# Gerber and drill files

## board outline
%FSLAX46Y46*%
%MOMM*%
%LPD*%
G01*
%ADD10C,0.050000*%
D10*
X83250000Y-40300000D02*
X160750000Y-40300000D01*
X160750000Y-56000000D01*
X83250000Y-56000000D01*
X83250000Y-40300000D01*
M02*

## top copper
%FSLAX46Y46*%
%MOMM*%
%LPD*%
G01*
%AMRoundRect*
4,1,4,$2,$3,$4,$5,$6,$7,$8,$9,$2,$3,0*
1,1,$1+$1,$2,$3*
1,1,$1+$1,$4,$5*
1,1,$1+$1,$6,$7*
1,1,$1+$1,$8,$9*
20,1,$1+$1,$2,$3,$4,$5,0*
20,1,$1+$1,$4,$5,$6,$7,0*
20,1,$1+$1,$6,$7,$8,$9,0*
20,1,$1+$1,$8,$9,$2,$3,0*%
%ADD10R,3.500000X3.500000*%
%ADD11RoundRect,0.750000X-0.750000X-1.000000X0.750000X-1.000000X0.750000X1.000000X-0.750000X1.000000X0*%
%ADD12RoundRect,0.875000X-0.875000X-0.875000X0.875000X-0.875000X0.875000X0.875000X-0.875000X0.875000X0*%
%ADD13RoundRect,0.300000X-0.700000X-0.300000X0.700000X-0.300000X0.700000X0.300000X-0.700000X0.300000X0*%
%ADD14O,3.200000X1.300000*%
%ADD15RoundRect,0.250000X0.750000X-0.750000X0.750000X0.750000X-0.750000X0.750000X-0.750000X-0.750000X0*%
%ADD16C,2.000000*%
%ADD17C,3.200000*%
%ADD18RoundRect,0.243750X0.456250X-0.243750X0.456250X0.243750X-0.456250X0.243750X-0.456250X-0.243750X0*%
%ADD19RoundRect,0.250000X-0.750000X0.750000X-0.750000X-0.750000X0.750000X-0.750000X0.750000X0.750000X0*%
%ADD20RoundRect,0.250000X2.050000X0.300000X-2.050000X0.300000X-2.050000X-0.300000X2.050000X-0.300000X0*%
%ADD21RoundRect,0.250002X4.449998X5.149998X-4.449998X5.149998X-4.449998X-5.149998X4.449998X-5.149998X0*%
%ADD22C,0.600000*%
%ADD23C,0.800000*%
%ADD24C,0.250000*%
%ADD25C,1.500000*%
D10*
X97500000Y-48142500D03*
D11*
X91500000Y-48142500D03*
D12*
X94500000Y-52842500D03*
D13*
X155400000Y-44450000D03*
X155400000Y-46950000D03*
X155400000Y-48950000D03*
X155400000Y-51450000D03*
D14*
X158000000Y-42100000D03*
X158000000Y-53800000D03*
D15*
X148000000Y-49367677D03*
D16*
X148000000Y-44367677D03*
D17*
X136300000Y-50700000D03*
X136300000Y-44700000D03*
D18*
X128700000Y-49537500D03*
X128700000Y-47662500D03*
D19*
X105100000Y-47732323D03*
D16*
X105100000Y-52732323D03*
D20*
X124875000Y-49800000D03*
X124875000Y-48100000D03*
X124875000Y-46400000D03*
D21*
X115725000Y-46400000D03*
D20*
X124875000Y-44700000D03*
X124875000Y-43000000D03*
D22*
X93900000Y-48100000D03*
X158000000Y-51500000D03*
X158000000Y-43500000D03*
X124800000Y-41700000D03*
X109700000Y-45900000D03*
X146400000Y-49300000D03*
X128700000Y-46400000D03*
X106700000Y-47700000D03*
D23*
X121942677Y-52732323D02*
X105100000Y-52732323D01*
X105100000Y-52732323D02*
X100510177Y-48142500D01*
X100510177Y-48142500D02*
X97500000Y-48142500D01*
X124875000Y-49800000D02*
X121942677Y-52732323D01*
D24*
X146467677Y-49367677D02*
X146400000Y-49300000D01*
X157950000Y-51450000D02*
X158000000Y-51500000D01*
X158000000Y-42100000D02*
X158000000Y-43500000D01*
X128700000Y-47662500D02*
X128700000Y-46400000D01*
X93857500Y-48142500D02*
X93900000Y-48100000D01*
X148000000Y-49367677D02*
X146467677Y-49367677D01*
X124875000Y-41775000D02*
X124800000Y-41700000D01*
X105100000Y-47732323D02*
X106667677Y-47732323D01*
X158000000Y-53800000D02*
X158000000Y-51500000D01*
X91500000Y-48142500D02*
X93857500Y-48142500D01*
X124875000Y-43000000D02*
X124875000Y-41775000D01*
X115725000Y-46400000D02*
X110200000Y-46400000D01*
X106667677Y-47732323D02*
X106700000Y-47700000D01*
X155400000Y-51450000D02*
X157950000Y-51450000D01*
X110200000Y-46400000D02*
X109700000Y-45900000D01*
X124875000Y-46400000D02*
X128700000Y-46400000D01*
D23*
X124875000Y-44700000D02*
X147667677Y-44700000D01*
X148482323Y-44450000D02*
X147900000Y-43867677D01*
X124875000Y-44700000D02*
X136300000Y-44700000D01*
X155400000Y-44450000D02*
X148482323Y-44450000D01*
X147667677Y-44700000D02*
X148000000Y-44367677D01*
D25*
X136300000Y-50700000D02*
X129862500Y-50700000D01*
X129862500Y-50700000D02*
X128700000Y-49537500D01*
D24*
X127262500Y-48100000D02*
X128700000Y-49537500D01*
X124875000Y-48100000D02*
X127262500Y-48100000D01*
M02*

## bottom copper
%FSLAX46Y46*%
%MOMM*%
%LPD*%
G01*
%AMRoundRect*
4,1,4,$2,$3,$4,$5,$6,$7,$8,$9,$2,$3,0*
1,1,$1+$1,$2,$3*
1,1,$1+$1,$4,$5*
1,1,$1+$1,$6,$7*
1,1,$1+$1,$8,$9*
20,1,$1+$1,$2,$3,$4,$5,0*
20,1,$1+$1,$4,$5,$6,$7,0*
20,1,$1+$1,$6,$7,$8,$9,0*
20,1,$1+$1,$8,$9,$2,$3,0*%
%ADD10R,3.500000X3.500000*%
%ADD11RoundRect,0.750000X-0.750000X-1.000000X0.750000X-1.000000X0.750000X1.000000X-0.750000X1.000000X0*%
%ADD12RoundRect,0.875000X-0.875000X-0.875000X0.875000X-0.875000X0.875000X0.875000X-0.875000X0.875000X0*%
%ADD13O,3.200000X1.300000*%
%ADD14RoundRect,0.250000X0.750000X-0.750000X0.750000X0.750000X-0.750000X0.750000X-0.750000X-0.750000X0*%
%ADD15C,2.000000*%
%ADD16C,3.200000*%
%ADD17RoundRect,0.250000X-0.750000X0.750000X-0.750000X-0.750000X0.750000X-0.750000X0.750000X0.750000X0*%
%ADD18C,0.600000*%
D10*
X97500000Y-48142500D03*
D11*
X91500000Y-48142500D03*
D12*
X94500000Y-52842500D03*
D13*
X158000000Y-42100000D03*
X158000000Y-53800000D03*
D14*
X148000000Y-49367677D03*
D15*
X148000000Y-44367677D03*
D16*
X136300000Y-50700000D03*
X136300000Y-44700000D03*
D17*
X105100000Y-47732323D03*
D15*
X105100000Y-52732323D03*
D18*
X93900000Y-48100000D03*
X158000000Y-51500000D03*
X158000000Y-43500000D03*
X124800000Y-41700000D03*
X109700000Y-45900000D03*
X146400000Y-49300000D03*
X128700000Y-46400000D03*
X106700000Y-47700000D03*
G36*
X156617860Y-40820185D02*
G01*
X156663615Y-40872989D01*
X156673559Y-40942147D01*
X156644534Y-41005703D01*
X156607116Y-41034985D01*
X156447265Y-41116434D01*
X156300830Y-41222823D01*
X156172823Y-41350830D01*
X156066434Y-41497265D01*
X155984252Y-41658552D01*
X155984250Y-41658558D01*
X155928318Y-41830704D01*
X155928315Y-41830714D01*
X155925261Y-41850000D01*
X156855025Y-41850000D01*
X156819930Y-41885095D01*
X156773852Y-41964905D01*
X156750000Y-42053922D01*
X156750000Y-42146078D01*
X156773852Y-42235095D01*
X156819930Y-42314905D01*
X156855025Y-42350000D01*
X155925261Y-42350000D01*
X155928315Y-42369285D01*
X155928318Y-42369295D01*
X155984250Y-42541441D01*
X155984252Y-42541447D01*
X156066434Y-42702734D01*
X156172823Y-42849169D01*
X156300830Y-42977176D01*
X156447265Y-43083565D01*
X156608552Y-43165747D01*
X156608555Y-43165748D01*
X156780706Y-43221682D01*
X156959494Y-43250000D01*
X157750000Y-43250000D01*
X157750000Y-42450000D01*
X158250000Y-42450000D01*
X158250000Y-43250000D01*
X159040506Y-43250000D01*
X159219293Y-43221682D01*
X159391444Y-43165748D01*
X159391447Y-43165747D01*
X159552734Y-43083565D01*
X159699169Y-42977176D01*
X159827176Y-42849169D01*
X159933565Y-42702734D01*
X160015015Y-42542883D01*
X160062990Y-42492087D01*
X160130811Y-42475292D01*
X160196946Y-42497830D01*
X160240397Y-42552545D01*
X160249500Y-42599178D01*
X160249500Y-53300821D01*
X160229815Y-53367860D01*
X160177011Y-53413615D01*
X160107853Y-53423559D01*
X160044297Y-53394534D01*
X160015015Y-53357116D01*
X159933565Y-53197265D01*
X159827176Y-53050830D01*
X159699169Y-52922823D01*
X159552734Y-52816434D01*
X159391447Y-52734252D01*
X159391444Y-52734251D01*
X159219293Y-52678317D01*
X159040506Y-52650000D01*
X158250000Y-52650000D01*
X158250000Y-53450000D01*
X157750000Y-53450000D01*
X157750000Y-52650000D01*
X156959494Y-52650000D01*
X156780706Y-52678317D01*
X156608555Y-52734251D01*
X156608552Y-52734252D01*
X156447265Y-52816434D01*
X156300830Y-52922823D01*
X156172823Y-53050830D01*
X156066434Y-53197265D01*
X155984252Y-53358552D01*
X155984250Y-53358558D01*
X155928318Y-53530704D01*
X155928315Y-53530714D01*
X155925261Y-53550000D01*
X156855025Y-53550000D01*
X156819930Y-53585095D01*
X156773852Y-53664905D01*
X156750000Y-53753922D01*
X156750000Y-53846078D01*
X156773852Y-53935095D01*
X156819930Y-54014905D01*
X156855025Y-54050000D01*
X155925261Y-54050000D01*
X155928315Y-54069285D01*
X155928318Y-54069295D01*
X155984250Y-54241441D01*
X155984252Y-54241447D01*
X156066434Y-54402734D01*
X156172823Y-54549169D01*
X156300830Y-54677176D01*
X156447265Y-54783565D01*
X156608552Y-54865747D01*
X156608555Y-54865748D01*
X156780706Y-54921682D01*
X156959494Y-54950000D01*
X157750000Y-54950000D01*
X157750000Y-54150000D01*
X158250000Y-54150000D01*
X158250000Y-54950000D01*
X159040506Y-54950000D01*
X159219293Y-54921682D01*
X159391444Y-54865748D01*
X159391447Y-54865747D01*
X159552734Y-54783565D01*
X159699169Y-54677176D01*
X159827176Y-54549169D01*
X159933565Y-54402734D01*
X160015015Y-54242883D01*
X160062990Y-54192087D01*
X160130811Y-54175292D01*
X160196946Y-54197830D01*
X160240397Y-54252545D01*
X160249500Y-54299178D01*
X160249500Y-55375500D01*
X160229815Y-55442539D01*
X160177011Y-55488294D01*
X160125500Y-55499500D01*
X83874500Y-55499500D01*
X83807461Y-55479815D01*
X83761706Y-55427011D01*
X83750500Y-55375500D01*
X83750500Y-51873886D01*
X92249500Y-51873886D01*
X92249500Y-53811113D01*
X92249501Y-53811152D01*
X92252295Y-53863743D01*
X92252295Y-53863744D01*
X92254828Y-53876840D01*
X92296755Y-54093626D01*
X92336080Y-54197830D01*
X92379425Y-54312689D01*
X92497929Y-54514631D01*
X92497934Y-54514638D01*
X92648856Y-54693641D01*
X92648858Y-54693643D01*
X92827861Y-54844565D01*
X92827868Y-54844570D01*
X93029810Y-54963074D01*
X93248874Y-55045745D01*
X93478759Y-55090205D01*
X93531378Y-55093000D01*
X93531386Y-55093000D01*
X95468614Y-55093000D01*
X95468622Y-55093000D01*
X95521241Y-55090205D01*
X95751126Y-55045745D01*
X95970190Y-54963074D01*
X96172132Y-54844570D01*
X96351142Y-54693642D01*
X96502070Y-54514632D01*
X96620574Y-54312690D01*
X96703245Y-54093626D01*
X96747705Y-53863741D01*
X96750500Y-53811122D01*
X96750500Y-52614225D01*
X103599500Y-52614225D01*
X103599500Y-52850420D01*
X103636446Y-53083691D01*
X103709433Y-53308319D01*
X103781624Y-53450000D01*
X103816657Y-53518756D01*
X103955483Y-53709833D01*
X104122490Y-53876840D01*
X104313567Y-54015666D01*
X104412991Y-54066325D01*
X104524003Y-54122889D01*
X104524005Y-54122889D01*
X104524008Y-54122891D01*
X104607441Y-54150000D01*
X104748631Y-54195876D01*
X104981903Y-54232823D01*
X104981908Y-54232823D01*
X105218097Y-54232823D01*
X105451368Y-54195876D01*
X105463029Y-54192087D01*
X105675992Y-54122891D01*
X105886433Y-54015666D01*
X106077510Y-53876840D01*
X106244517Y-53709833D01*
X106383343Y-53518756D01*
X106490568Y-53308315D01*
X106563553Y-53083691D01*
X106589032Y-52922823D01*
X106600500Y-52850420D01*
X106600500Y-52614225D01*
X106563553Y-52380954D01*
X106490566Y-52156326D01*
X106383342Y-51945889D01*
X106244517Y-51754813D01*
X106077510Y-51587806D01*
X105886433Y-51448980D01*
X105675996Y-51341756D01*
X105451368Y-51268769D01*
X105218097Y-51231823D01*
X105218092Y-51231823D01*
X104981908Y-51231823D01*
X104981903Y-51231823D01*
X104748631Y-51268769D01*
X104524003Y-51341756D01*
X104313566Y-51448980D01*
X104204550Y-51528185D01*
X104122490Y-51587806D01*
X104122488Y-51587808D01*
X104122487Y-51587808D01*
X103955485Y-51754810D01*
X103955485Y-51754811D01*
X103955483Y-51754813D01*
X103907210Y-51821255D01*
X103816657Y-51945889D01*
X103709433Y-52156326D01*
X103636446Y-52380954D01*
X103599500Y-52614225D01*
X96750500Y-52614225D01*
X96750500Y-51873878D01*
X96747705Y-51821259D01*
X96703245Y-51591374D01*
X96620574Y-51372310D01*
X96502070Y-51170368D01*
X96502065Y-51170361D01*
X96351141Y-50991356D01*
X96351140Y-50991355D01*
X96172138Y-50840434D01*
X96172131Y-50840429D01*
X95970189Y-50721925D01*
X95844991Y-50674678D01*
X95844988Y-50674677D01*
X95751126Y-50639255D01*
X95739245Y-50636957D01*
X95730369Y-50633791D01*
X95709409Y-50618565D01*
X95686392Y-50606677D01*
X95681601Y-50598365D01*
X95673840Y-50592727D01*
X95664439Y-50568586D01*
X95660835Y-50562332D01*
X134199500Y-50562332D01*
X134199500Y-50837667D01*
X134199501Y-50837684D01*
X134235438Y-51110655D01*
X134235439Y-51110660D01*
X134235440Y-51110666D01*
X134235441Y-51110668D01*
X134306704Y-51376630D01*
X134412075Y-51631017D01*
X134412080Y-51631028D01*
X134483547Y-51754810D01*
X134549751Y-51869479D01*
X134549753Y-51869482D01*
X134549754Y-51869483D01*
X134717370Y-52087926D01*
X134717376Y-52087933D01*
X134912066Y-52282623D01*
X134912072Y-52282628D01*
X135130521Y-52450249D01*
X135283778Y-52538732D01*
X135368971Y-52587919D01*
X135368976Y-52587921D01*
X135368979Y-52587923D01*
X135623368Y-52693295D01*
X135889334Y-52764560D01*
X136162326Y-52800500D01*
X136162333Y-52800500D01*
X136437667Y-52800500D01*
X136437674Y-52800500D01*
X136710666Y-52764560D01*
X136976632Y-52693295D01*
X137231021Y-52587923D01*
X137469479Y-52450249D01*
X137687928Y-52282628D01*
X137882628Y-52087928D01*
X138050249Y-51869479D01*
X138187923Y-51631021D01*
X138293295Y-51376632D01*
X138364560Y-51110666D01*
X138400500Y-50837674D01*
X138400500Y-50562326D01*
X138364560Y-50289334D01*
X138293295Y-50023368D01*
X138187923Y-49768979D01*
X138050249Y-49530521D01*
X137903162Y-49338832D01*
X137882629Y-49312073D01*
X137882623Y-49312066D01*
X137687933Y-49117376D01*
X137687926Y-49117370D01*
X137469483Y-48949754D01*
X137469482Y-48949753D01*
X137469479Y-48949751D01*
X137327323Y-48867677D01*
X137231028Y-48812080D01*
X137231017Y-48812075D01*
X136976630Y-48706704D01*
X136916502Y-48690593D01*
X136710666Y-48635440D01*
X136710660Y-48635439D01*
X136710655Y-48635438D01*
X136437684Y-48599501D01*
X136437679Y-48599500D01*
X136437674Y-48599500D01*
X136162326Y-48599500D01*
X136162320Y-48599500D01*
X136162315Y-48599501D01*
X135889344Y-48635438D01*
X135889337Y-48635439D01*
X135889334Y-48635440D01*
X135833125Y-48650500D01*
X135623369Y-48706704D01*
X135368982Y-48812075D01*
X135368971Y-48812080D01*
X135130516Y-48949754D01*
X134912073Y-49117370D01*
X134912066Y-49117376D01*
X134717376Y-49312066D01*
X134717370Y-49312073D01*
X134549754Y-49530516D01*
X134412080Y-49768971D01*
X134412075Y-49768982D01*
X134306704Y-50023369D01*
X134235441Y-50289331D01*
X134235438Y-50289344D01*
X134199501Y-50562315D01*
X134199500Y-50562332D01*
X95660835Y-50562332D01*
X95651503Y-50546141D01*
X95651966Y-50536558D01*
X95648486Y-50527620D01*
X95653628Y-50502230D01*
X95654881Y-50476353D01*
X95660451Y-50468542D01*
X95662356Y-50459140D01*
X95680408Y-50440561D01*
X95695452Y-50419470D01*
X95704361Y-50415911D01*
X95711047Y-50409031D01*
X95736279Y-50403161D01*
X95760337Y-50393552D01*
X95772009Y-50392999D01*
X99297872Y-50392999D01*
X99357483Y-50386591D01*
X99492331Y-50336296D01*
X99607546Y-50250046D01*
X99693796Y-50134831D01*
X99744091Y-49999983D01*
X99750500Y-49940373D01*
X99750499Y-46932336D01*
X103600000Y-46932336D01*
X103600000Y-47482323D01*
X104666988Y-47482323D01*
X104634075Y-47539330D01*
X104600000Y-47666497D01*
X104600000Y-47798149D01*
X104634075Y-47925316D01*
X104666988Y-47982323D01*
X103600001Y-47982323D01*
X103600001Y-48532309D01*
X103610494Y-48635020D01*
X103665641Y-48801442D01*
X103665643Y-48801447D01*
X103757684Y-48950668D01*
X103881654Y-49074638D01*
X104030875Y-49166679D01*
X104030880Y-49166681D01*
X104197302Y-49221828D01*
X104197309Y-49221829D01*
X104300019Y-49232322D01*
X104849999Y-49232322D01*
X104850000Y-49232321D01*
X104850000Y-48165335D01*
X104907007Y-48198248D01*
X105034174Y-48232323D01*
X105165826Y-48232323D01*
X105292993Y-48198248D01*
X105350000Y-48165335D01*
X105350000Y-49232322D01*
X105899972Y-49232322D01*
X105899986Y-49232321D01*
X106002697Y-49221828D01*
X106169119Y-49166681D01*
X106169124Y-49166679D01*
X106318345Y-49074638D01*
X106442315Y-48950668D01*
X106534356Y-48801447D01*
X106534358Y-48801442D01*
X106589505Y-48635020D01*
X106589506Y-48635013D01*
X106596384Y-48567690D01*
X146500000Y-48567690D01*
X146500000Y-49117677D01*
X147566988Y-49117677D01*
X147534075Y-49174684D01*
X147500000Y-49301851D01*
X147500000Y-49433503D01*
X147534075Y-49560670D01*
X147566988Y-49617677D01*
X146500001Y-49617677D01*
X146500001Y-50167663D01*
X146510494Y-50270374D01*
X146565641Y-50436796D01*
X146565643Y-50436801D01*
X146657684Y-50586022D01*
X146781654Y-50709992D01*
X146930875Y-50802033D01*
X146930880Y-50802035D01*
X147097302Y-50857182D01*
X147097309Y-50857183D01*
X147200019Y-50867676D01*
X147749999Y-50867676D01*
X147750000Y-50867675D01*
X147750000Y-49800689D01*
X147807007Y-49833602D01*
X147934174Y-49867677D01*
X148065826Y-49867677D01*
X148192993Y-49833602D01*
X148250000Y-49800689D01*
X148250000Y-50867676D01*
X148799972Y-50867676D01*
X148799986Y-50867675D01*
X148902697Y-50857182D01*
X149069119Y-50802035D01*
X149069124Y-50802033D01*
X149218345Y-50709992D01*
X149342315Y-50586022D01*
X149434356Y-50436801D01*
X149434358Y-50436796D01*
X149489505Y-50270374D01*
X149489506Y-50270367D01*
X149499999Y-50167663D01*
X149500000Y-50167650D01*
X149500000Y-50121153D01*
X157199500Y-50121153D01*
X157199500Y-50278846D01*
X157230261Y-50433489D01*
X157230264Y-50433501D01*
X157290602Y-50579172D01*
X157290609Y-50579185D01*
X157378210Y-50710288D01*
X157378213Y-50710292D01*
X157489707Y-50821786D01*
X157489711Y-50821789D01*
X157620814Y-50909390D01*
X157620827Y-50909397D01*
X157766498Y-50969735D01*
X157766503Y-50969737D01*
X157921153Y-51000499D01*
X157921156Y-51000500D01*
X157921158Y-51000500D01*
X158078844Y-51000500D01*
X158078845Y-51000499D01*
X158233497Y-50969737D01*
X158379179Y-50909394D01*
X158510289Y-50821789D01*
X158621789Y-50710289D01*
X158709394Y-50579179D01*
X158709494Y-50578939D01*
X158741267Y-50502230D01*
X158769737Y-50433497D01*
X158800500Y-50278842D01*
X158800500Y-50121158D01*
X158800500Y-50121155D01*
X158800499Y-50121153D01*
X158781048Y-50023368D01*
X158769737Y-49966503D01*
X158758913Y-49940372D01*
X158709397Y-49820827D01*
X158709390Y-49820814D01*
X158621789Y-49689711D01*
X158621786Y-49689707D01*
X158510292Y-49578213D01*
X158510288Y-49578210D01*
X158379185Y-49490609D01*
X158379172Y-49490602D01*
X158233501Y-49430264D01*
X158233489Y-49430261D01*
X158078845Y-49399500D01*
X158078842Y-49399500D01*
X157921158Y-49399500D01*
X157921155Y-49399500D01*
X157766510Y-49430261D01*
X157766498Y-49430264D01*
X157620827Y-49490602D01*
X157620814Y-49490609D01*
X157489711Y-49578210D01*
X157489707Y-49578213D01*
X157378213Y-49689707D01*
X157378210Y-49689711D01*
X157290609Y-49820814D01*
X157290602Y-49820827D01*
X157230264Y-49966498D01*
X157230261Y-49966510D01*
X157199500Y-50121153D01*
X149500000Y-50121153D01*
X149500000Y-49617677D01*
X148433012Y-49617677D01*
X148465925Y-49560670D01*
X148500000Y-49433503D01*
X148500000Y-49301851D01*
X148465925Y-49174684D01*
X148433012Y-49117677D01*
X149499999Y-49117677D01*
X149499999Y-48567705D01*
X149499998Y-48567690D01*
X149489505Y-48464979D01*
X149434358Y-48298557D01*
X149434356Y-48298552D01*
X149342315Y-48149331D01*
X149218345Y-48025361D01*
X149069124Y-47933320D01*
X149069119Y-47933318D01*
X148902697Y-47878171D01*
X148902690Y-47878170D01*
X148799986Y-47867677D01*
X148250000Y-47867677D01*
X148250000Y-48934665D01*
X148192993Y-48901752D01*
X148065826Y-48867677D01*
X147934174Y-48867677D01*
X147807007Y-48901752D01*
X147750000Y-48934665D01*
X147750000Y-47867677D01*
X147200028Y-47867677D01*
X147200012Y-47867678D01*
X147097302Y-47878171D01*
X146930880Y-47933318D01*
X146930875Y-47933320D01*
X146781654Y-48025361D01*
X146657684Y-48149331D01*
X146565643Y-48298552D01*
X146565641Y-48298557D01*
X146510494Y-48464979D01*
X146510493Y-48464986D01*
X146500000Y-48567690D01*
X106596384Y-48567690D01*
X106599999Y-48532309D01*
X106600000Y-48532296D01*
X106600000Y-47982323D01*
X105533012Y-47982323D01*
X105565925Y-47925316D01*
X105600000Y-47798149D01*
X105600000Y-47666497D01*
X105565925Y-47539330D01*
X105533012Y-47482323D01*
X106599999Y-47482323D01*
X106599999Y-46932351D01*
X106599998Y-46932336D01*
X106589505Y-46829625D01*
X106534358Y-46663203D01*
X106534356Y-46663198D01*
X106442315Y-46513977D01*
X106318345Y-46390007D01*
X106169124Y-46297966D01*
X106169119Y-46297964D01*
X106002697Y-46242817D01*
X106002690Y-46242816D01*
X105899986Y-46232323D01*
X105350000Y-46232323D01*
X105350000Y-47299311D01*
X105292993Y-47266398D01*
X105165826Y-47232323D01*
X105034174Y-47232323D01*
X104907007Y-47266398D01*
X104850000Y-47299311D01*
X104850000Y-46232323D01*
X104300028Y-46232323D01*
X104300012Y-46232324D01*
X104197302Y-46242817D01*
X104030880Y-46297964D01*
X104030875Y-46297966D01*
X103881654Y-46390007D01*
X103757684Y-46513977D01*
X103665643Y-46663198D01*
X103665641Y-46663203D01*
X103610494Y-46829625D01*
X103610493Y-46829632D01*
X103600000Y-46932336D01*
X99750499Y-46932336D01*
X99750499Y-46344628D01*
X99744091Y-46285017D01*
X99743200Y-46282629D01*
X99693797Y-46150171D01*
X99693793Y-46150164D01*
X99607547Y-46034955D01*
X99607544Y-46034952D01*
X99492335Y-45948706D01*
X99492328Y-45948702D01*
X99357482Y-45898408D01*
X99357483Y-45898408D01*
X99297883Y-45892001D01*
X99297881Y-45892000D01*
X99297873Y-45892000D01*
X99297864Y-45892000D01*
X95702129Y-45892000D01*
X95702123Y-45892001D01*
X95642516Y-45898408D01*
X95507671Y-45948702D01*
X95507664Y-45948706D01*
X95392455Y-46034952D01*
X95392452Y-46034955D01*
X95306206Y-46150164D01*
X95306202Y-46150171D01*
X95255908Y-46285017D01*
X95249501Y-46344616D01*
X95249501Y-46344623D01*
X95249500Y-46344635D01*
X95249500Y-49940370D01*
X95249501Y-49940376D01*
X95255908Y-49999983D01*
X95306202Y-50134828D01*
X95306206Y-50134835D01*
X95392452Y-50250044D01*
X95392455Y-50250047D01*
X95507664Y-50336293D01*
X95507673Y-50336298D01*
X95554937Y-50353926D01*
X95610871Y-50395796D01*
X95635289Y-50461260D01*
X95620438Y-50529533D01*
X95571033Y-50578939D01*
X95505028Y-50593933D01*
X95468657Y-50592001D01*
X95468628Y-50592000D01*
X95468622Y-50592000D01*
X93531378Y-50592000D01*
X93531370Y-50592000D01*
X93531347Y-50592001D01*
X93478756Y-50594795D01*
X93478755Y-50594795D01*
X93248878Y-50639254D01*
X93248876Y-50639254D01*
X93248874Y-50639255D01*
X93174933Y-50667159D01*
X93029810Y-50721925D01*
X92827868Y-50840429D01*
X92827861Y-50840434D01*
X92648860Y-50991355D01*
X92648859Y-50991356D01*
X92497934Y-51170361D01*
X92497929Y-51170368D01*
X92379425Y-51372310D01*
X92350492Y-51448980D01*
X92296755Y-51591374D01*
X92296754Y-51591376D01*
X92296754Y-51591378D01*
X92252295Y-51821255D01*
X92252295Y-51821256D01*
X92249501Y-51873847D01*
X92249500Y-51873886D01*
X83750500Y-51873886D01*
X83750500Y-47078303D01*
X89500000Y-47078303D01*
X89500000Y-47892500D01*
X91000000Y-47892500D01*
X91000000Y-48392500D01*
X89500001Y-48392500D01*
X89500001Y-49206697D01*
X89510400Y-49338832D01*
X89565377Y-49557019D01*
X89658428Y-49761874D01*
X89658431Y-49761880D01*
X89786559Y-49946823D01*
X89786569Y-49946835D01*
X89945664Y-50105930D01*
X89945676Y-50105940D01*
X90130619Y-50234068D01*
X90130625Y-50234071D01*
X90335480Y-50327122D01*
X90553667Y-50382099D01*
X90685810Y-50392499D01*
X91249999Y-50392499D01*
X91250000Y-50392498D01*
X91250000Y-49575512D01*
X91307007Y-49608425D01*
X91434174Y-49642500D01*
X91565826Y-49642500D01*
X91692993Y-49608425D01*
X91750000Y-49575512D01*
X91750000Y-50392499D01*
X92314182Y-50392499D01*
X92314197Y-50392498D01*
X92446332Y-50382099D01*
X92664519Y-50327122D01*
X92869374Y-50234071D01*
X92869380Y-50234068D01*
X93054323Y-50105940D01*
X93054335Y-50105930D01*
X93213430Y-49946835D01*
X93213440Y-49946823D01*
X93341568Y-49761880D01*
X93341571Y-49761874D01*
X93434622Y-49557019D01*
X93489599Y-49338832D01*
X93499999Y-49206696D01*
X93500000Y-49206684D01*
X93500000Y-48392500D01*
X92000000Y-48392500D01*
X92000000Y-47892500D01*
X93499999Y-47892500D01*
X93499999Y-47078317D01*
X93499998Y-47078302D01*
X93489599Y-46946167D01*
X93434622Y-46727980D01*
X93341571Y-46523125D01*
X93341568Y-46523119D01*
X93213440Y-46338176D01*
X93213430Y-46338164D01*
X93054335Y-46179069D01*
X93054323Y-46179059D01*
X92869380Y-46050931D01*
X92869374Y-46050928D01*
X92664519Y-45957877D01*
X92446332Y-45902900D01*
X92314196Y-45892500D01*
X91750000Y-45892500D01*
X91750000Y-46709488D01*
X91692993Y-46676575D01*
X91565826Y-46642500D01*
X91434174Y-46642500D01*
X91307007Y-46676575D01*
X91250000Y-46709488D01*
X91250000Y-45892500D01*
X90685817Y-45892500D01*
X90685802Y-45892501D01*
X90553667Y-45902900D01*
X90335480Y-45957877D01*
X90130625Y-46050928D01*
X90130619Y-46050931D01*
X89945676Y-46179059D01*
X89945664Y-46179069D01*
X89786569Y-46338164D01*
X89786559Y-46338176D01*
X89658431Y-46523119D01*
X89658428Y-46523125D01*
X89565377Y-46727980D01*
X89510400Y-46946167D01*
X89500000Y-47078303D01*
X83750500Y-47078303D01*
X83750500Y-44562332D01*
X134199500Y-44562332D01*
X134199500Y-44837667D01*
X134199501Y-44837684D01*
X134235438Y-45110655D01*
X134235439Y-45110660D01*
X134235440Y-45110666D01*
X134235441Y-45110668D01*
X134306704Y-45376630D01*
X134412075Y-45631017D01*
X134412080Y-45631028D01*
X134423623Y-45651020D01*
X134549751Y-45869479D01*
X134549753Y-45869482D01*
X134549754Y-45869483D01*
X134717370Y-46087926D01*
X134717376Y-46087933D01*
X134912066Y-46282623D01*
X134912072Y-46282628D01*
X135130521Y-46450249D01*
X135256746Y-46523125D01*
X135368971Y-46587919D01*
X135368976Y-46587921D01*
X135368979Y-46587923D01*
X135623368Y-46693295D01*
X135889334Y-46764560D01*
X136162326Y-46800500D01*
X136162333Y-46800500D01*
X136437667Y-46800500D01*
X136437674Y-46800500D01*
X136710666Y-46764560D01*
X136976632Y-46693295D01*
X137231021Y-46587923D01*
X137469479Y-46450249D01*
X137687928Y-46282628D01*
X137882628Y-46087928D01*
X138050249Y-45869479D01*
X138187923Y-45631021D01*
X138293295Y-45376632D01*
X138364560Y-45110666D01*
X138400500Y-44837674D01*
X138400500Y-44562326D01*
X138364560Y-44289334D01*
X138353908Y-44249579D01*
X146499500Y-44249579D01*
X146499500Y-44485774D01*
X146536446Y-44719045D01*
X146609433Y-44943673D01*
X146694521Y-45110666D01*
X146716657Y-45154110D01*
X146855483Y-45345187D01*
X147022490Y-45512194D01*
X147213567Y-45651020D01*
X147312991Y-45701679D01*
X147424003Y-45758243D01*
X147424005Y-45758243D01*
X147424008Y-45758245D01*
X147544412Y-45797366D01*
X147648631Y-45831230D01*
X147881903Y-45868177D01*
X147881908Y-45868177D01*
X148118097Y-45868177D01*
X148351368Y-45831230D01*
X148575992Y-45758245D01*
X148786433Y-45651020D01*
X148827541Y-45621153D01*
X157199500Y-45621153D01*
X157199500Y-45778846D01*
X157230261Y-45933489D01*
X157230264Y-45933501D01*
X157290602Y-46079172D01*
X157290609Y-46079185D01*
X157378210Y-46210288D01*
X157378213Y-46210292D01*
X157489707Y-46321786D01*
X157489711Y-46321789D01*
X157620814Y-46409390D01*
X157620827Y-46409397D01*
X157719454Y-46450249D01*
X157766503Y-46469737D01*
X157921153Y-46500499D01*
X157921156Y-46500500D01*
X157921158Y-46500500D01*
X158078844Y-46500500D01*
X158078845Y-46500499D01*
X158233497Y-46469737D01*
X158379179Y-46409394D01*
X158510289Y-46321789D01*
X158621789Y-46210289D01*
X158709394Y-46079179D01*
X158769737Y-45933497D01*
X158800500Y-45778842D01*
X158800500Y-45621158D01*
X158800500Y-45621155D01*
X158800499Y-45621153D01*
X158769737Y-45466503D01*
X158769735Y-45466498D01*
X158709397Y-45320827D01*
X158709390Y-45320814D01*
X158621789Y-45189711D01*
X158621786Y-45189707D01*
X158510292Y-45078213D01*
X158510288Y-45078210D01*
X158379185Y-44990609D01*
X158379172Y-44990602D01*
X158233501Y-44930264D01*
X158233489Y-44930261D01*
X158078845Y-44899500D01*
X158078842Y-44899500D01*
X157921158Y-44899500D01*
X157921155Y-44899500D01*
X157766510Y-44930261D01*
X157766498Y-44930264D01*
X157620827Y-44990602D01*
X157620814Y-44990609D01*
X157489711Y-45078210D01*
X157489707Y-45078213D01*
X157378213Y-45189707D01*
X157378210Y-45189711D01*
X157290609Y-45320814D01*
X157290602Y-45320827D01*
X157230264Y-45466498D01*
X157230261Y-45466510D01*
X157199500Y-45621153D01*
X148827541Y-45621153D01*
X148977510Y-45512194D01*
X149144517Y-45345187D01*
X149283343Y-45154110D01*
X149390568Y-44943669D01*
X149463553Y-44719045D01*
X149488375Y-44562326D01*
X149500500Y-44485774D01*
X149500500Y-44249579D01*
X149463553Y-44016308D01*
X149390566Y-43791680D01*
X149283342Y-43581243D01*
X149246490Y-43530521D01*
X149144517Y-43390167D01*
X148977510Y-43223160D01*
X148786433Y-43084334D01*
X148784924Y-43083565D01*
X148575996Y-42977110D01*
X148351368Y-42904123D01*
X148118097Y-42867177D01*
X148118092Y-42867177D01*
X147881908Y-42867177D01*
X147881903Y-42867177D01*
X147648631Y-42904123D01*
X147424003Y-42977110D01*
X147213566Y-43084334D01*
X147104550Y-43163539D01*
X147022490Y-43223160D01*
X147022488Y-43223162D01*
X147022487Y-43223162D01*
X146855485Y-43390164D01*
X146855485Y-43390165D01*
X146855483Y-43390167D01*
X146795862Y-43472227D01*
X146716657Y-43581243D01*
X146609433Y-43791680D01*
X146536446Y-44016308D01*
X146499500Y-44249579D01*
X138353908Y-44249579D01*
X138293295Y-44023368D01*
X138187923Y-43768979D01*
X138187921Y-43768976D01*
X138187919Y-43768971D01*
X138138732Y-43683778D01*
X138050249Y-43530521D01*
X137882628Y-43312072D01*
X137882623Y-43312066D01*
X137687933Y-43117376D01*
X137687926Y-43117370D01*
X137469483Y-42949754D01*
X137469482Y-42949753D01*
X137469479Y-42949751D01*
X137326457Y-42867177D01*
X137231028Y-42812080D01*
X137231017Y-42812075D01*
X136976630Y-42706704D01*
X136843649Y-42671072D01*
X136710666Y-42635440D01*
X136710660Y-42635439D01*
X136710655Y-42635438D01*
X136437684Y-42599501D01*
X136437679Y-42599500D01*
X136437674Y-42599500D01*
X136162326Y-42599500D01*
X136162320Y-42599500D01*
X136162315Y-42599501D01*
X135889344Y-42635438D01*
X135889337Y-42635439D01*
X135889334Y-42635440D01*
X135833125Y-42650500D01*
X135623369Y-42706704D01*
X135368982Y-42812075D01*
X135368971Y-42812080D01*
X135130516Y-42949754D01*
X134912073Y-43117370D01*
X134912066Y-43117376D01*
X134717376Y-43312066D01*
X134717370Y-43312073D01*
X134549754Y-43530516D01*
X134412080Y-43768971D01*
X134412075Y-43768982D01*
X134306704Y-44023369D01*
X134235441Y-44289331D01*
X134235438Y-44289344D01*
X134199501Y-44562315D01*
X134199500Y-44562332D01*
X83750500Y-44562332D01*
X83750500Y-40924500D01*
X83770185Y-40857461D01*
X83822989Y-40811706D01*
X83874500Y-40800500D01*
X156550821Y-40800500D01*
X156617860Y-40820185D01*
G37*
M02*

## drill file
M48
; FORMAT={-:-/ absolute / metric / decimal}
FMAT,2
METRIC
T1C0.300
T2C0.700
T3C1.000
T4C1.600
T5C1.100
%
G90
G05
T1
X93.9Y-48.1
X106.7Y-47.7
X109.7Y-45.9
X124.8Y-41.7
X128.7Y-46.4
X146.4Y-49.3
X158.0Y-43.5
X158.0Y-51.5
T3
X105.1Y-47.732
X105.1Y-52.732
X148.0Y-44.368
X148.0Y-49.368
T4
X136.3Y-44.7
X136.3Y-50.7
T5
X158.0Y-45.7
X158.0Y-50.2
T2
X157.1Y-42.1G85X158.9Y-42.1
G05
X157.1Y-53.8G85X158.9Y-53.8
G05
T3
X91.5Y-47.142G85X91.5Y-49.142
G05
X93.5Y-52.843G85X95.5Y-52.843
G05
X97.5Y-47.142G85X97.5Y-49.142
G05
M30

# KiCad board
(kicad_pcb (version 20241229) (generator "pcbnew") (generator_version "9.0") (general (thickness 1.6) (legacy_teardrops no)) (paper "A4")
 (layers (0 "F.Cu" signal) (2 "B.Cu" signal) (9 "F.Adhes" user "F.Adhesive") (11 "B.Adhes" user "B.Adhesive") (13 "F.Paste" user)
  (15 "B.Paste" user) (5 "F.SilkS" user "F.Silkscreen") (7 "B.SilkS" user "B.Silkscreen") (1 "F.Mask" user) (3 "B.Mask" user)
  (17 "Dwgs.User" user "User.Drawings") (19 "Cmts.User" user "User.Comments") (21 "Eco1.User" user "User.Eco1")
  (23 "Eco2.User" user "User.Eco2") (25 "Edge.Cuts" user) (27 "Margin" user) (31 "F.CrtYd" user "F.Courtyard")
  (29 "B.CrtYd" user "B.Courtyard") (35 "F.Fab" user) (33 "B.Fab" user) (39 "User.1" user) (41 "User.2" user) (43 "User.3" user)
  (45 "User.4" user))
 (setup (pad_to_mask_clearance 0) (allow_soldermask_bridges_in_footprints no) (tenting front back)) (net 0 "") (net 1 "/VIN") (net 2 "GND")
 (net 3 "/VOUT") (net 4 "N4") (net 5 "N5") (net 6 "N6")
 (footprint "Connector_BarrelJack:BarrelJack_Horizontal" (layer "F.Cu") (at 97.5 48.1425)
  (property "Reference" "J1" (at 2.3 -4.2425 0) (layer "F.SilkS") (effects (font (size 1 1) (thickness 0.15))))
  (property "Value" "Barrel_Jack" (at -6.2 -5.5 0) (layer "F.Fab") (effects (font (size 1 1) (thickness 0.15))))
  (pad "1" thru_hole rect (at 0 0) (size 3.5 3.5) (drill oval 1 3) (layers "*.Cu" "*.Mask") (remove_unused_layers no) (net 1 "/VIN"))
  (pad "2" thru_hole roundrect (at -6 0) (size 3 3.5) (drill oval 1 3) (layers "*.Cu" "*.Mask") (remove_unused_layers no)
   (roundrect_rratio 0.25) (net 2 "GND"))
  (pad "3" thru_hole roundrect (at -3 4.7) (size 3.5 3.5) (drill oval 3 1) (layers "*.Cu" "*.Mask") (remove_unused_layers no)
   (roundrect_rratio 0.25)))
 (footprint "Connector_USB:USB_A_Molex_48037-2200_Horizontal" (layer "F.Cu") (at 166.375 47.95)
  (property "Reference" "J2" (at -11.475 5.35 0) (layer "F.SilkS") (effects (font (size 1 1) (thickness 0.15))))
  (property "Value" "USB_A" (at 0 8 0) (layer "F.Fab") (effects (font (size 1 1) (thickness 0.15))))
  (pad "" np_thru_hole circle (at -8.375 -2.25) (size 1.1 1.1) (drill 1.1) (layers "*.Mask"))
  (pad "" np_thru_hole circle (at -8.375 2.25) (size 1.1 1.1) (drill 1.1) (layers "*.Mask"))
  (pad "1" smd roundrect (at -10.975 -3.5) (size 2 1.2) (layers "F.Cu" "F.Mask" "F.Paste") (roundrect_rratio 0.25) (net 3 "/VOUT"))
  (pad "2" smd roundrect (at -10.975 -1) (size 2 1.2) (layers "F.Cu" "F.Mask" "F.Paste") (roundrect_rratio 0.25) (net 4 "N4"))
  (pad "3" smd roundrect (at -10.975 1) (size 2 1.2) (layers "F.Cu" "F.Mask" "F.Paste") (roundrect_rratio 0.25) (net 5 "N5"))
  (pad "4" smd roundrect (at -10.975 3.5) (size 2 1.2) (layers "F.Cu" "F.Mask" "F.Paste") (roundrect_rratio 0.25) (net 2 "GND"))
  (pad "5" thru_hole oval (at -8.375 -5.85) (size 3.2 1.3) (drill oval 2.5 0.7) (layers "*.Cu" "*.Mask") (remove_unused_layers no)
   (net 2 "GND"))
  (pad "5" thru_hole oval (at -8.375 5.85) (size 3.2 1.3) (drill oval 2.5 0.7) (layers "*.Cu" "*.Mask") (remove_unused_layers no)
   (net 2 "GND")))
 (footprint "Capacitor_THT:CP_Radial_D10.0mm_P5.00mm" (layer "F.Cu") (at 148 49.367677 90)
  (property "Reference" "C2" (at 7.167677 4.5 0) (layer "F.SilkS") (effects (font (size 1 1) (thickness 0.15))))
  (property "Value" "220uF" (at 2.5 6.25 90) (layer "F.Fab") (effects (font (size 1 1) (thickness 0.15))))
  (pad "1" thru_hole roundrect (at 0 0 90) (size 2 2) (drill 1) (layers "*.Cu" "*.Mask") (remove_unused_layers no) (roundrect_rratio 0.125)
   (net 2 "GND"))
  (pad "2" thru_hole circle (at 5 0 90) (size 2 2) (drill 1) (layers "*.Cu" "*.Mask") (remove_unused_layers no) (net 3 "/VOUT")))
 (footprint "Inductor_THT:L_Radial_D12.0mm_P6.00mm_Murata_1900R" (layer "F.Cu") (at 136.3 50.7 90)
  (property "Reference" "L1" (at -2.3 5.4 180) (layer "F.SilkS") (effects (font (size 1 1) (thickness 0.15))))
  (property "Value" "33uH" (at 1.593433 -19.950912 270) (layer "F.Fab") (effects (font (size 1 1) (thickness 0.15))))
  (pad "1" thru_hole circle (at 0 0 90) (size 3.2 3.2) (drill 1.6) (layers "*.Cu" "*.Mask") (remove_unused_layers no) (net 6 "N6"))
  (pad "2" thru_hole circle (at 6 0 90) (size 3.2 3.2) (drill 1.6) (layers "*.Cu" "*.Mask") (remove_unused_layers no) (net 3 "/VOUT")))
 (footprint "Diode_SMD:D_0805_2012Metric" (layer "F.Cu") (at 128.7 48.6 90)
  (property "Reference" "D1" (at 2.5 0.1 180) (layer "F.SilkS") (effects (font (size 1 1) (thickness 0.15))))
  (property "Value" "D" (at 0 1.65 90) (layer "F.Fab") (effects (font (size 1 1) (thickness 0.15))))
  (pad "1" smd roundrect (at -0.9375 0 90) (size 0.975 1.4) (layers "F.Cu" "F.Mask" "F.Paste") (roundrect_rratio 0.25) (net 6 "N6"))
  (pad "2" smd roundrect (at 0.9375 0 90) (size 0.975 1.4) (layers "F.Cu" "F.Mask" "F.Paste") (roundrect_rratio 0.25) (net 2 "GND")))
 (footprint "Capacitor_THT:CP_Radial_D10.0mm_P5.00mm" (layer "F.Cu") (at 105.1 47.732323 -90)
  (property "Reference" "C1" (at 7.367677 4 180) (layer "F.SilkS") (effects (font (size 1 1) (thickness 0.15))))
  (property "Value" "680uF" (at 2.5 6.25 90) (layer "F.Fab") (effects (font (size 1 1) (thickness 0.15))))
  (pad "1" thru_hole roundrect (at 0 0 270) (size 2 2) (drill 1) (layers "*.Cu" "*.Mask") (remove_unused_layers no) (roundrect_rratio 0.125)
   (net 2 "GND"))
  (pad "2" thru_hole circle (at 5 0 270) (size 2 2) (drill 1) (layers "*.Cu" "*.Mask") (remove_unused_layers no) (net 1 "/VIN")))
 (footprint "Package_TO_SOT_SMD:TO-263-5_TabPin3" (layer "F.Cu") (at 117.225 46.4 180)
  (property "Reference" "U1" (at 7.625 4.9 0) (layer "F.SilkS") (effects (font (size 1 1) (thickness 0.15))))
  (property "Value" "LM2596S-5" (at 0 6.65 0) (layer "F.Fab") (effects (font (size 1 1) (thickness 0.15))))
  (pad "" smd roundrect (at -0.925 -2.775 180) (size 4.55 5.25) (layers "F.Paste") (roundrect_rratio 0.054945))
  (pad "" smd roundrect (at -0.925 2.775 180) (size 4.55 5.25) (layers "F.Paste") (roundrect_rratio 0.054945))
  (pad "" smd roundrect (at 3.925 -2.775 180) (size 4.55 5.25) (layers "F.Paste") (roundrect_rratio 0.054945))
  (pad "" smd roundrect (at 3.925 2.775 180) (size 4.55 5.25) (layers "F.Paste") (roundrect_rratio 0.054945))
  (pad "1" smd roundrect (at -7.65 -3.4 180) (size 4.6 1.1) (layers "F.Cu" "F.Mask" "F.Paste") (roundrect_rratio 0.227273) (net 1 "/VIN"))
  (pad "2" smd roundrect (at -7.65 -1.7 180) (size 4.6 1.1) (layers "F.Cu" "F.Mask" "F.Paste") (roundrect_rratio 0.227273) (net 6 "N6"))
  (pad "3" smd roundrect (at -7.65 0 180) (size 4.6 1.1) (layers "F.Cu" "F.Mask" "F.Paste") (roundrect_rratio 0.227273) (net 2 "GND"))
  (pad "3" smd roundrect (at 1.5 0 180) (size 9.4 10.8) (layers "F.Cu" "F.Mask") (roundrect_rratio 0.026596) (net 2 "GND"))
  (pad "4" smd roundrect (at -7.65 1.7 180) (size 4.6 1.1) (layers "F.Cu" "F.Mask" "F.Paste") (roundrect_rratio 0.227273) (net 3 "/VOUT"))
  (pad "5" smd roundrect (at -7.65 3.4 180) (size 4.6 1.1) (layers "F.Cu" "F.Mask" "F.Paste") (roundrect_rratio 0.227273) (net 2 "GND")))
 (gr_rect (start 83.25 40.3) (end 160.75 56) (stroke (width 0.05) (type default)) (fill no) (layer "Edge.Cuts"))
 (segment (start 121.942677 52.732323) (end 105.1 52.732323) (width 0.8) (layer "F.Cu") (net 1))
 (segment (start 105.1 52.732323) (end 100.510177 48.1425) (width 0.8) (layer "F.Cu") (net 1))
 (segment (start 100.510177 48.1425) (end 97.5 48.1425) (width 0.8) (layer "F.Cu") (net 1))
 (segment (start 124.875 49.8) (end 121.942677 52.732323) (width 0.8) (layer "F.Cu") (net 1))
 (segment (start 146.467677 49.367677) (end 146.4 49.3) (width 0.25) (layer "F.Cu") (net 2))
 (segment (start 157.95 51.45) (end 158 51.5) (width 0.25) (layer "F.Cu") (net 2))
 (segment (start 158 42.1) (end 158 43.5) (width 0.25) (layer "F.Cu") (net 2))
 (segment (start 128.7 47.6625) (end 128.7 46.4) (width 0.25) (layer "F.Cu") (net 2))
 (segment (start 93.8575 48.1425) (end 93.9 48.1) (width 0.25) (layer "F.Cu") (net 2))
 (segment (start 148 49.367677) (end 146.467677 49.367677) (width 0.25) (layer "F.Cu") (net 2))
 (segment (start 124.875 41.775) (end 124.8 41.7) (width 0.25) (layer "F.Cu") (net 2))
 (segment (start 105.1 47.732323) (end 106.667677 47.732323) (width 0.25) (layer "F.Cu") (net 2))
 (segment (start 158 53.8) (end 158 51.5) (width 0.25) (layer "F.Cu") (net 2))
 (segment (start 91.5 48.1425) (end 93.8575 48.1425) (width 0.25) (layer "F.Cu") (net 2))
 (segment (start 124.875 43) (end 124.875 41.775) (width 0.25) (layer "F.Cu") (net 2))
 (segment (start 115.725 46.4) (end 110.2 46.4) (width 0.25) (layer "F.Cu") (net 2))
 (segment (start 106.667677 47.732323) (end 106.7 47.7) (width 0.25) (layer "F.Cu") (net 2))
 (segment (start 155.4 51.45) (end 157.95 51.45) (width 0.25) (layer "F.Cu") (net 2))
 (segment (start 110.2 46.4) (end 109.7 45.9) (width 0.25) (layer "F.Cu") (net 2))
 (segment (start 124.875 46.4) (end 128.7 46.4) (width 0.25) (layer "F.Cu") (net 2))
 (via (at 93.9 48.1) (size 0.6) (drill 0.3) (layers "F.Cu" "B.Cu") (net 2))
 (via (at 158 51.5) (size 0.6) (drill 0.3) (layers "F.Cu" "B.Cu") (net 2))
 (via (at 158 43.5) (size 0.6) (drill 0.3) (layers "F.Cu" "B.Cu") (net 2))
 (via (at 124.8 41.7) (size 0.6) (drill 0.3) (layers "F.Cu" "B.Cu") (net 2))
 (via (at 109.7 45.9) (size 0.6) (drill 0.3) (layers "F.Cu" "B.Cu") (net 2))
 (via (at 146.4 49.3) (size 0.6) (drill 0.3) (layers "F.Cu" "B.Cu") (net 2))
 (via (at 128.7 46.4) (size 0.6) (drill 0.3) (layers "F.Cu" "B.Cu") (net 2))
 (via (at 106.7 47.7) (size 0.6) (drill 0.3) (layers "F.Cu" "B.Cu") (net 2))
 (segment (start 124.875 44.7) (end 147.667677 44.7) (width 0.8) (layer "F.Cu") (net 3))
 (segment (start 148.482323 44.45) (end 147.9 43.867677) (width 0.8) (layer "F.Cu") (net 3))
 (segment (start 124.875 44.7) (end 136.3 44.7) (width 0.8) (layer "F.Cu") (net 3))
 (segment (start 155.4 44.45) (end 148.482323 44.45) (width 0.8) (layer "F.Cu") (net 3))
 (segment (start 147.667677 44.7) (end 148 44.367677) (width 0.8) (layer "F.Cu") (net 3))
 (segment (start 136.3 50.7) (end 129.8625 50.7) (width 1.5) (layer "F.Cu") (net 6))
 (segment (start 129.8625 50.7) (end 128.7 49.5375) (width 1.5) (layer "F.Cu") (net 6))
 (segment (start 127.2625 48.1) (end 128.7 49.5375) (width 0.25) (layer "F.Cu") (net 6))
 (segment (start 124.875 48.1) (end 127.2625 48.1) (width 0.25) (layer "F.Cu") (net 6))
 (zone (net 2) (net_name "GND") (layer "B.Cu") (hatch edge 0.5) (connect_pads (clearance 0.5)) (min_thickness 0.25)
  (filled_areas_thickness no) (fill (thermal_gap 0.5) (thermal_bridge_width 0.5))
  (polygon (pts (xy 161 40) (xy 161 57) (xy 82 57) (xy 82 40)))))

